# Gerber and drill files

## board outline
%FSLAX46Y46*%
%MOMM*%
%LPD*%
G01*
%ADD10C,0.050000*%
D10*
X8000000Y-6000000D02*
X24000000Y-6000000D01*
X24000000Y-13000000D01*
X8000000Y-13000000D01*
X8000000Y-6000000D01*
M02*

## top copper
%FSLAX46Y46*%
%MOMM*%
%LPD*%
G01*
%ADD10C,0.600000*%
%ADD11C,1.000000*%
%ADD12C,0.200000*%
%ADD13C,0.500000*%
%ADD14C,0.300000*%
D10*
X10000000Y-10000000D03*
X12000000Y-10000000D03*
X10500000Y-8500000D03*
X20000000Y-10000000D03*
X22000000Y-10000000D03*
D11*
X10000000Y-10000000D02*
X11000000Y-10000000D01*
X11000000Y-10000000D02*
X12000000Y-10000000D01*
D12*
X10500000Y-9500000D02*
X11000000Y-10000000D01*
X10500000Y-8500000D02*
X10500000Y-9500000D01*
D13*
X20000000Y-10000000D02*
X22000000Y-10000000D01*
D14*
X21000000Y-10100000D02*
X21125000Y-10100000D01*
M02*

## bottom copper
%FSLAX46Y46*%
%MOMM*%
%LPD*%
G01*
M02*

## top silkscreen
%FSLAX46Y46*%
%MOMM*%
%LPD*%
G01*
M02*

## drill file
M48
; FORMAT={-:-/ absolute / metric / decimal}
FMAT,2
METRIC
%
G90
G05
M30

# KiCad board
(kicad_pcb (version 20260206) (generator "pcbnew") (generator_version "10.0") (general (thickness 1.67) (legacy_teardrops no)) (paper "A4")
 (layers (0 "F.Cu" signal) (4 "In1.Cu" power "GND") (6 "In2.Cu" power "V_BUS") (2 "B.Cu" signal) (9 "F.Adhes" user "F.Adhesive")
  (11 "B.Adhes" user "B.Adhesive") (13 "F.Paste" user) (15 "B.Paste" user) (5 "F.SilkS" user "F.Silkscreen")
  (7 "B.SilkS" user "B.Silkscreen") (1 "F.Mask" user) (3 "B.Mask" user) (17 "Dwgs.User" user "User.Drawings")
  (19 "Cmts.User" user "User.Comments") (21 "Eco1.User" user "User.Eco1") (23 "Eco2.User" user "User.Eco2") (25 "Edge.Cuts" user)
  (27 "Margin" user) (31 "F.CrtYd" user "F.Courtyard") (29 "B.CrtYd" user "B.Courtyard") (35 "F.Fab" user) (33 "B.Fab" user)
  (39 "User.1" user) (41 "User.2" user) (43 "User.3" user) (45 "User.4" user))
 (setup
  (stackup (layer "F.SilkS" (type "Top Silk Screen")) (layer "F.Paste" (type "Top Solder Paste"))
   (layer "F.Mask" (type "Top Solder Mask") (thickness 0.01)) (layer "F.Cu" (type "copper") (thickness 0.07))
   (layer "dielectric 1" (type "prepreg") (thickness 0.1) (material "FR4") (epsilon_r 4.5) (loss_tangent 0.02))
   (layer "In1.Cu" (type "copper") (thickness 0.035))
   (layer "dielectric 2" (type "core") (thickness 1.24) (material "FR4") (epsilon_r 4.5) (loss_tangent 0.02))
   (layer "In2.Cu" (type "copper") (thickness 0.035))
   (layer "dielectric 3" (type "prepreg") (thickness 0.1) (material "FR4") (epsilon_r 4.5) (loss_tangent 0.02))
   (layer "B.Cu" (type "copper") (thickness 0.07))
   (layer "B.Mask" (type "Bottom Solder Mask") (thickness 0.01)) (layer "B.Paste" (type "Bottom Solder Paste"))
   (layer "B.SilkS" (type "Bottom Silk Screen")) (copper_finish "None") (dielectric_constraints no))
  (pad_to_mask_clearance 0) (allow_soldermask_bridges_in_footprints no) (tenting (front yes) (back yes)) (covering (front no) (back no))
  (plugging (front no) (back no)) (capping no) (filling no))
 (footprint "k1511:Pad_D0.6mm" (layer "F.Cu") (at 10 10)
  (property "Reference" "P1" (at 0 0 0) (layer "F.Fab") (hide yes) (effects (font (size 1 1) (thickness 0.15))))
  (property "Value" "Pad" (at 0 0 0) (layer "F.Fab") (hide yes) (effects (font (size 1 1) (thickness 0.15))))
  (pad "1" smd circle (at 0 0) (size 0.6 0.6) (layers "F.Cu" "F.Mask") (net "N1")))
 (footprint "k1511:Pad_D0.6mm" (layer "F.Cu") (at 12 10)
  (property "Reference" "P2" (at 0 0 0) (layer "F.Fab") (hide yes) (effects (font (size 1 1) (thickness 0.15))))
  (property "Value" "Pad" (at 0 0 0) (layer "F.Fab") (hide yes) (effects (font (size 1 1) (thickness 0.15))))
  (pad "1" smd circle (at 0 0) (size 0.6 0.6) (layers "F.Cu" "F.Mask") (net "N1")))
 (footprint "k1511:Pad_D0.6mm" (layer "F.Cu") (at 10.5 8.5)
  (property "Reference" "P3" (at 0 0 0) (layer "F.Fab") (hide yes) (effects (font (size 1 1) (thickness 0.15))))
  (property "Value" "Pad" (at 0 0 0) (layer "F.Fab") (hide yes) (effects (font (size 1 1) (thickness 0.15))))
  (pad "1" smd circle (at 0 0) (size 0.6 0.6) (layers "F.Cu" "F.Mask") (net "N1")))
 (segment (start 10 10) (end 11 10) (width 1) (layer "F.Cu") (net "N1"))
 (segment (start 11 10) (end 12 10) (width 1) (layer "F.Cu") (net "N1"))
 (segment (start 10.5 9.5) (end 11 10) (width 0.2) (layer "F.Cu") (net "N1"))
 (segment (start 10.5 8.5) (end 10.5 9.5) (width 0.2) (layer "F.Cu") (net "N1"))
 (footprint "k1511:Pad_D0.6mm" (layer "F.Cu") (at 20 10)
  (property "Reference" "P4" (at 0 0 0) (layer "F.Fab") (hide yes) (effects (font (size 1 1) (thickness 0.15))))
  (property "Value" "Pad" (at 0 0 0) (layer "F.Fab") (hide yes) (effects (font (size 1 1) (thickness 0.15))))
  (pad "1" smd circle (at 0 0) (size 0.6 0.6) (layers "F.Cu" "F.Mask") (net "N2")))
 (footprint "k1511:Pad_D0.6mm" (layer "F.Cu") (at 22 10)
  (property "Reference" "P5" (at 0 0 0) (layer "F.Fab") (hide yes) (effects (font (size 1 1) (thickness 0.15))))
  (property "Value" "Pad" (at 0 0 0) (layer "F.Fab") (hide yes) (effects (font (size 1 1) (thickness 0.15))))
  (pad "1" smd circle (at 0 0) (size 0.6 0.6) (layers "F.Cu" "F.Mask") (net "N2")))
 (segment (start 20 10) (end 22 10) (width 0.5) (layer "F.Cu") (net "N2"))
 (segment (start 21 10.1) (end 21.125 10.1) (width 0.3) (layer "F.Cu") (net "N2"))
 (gr_rect (start 8 6) (end 24 13) (stroke (width 0.05) (type solid)) (fill no) (layer "Edge.Cuts")))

